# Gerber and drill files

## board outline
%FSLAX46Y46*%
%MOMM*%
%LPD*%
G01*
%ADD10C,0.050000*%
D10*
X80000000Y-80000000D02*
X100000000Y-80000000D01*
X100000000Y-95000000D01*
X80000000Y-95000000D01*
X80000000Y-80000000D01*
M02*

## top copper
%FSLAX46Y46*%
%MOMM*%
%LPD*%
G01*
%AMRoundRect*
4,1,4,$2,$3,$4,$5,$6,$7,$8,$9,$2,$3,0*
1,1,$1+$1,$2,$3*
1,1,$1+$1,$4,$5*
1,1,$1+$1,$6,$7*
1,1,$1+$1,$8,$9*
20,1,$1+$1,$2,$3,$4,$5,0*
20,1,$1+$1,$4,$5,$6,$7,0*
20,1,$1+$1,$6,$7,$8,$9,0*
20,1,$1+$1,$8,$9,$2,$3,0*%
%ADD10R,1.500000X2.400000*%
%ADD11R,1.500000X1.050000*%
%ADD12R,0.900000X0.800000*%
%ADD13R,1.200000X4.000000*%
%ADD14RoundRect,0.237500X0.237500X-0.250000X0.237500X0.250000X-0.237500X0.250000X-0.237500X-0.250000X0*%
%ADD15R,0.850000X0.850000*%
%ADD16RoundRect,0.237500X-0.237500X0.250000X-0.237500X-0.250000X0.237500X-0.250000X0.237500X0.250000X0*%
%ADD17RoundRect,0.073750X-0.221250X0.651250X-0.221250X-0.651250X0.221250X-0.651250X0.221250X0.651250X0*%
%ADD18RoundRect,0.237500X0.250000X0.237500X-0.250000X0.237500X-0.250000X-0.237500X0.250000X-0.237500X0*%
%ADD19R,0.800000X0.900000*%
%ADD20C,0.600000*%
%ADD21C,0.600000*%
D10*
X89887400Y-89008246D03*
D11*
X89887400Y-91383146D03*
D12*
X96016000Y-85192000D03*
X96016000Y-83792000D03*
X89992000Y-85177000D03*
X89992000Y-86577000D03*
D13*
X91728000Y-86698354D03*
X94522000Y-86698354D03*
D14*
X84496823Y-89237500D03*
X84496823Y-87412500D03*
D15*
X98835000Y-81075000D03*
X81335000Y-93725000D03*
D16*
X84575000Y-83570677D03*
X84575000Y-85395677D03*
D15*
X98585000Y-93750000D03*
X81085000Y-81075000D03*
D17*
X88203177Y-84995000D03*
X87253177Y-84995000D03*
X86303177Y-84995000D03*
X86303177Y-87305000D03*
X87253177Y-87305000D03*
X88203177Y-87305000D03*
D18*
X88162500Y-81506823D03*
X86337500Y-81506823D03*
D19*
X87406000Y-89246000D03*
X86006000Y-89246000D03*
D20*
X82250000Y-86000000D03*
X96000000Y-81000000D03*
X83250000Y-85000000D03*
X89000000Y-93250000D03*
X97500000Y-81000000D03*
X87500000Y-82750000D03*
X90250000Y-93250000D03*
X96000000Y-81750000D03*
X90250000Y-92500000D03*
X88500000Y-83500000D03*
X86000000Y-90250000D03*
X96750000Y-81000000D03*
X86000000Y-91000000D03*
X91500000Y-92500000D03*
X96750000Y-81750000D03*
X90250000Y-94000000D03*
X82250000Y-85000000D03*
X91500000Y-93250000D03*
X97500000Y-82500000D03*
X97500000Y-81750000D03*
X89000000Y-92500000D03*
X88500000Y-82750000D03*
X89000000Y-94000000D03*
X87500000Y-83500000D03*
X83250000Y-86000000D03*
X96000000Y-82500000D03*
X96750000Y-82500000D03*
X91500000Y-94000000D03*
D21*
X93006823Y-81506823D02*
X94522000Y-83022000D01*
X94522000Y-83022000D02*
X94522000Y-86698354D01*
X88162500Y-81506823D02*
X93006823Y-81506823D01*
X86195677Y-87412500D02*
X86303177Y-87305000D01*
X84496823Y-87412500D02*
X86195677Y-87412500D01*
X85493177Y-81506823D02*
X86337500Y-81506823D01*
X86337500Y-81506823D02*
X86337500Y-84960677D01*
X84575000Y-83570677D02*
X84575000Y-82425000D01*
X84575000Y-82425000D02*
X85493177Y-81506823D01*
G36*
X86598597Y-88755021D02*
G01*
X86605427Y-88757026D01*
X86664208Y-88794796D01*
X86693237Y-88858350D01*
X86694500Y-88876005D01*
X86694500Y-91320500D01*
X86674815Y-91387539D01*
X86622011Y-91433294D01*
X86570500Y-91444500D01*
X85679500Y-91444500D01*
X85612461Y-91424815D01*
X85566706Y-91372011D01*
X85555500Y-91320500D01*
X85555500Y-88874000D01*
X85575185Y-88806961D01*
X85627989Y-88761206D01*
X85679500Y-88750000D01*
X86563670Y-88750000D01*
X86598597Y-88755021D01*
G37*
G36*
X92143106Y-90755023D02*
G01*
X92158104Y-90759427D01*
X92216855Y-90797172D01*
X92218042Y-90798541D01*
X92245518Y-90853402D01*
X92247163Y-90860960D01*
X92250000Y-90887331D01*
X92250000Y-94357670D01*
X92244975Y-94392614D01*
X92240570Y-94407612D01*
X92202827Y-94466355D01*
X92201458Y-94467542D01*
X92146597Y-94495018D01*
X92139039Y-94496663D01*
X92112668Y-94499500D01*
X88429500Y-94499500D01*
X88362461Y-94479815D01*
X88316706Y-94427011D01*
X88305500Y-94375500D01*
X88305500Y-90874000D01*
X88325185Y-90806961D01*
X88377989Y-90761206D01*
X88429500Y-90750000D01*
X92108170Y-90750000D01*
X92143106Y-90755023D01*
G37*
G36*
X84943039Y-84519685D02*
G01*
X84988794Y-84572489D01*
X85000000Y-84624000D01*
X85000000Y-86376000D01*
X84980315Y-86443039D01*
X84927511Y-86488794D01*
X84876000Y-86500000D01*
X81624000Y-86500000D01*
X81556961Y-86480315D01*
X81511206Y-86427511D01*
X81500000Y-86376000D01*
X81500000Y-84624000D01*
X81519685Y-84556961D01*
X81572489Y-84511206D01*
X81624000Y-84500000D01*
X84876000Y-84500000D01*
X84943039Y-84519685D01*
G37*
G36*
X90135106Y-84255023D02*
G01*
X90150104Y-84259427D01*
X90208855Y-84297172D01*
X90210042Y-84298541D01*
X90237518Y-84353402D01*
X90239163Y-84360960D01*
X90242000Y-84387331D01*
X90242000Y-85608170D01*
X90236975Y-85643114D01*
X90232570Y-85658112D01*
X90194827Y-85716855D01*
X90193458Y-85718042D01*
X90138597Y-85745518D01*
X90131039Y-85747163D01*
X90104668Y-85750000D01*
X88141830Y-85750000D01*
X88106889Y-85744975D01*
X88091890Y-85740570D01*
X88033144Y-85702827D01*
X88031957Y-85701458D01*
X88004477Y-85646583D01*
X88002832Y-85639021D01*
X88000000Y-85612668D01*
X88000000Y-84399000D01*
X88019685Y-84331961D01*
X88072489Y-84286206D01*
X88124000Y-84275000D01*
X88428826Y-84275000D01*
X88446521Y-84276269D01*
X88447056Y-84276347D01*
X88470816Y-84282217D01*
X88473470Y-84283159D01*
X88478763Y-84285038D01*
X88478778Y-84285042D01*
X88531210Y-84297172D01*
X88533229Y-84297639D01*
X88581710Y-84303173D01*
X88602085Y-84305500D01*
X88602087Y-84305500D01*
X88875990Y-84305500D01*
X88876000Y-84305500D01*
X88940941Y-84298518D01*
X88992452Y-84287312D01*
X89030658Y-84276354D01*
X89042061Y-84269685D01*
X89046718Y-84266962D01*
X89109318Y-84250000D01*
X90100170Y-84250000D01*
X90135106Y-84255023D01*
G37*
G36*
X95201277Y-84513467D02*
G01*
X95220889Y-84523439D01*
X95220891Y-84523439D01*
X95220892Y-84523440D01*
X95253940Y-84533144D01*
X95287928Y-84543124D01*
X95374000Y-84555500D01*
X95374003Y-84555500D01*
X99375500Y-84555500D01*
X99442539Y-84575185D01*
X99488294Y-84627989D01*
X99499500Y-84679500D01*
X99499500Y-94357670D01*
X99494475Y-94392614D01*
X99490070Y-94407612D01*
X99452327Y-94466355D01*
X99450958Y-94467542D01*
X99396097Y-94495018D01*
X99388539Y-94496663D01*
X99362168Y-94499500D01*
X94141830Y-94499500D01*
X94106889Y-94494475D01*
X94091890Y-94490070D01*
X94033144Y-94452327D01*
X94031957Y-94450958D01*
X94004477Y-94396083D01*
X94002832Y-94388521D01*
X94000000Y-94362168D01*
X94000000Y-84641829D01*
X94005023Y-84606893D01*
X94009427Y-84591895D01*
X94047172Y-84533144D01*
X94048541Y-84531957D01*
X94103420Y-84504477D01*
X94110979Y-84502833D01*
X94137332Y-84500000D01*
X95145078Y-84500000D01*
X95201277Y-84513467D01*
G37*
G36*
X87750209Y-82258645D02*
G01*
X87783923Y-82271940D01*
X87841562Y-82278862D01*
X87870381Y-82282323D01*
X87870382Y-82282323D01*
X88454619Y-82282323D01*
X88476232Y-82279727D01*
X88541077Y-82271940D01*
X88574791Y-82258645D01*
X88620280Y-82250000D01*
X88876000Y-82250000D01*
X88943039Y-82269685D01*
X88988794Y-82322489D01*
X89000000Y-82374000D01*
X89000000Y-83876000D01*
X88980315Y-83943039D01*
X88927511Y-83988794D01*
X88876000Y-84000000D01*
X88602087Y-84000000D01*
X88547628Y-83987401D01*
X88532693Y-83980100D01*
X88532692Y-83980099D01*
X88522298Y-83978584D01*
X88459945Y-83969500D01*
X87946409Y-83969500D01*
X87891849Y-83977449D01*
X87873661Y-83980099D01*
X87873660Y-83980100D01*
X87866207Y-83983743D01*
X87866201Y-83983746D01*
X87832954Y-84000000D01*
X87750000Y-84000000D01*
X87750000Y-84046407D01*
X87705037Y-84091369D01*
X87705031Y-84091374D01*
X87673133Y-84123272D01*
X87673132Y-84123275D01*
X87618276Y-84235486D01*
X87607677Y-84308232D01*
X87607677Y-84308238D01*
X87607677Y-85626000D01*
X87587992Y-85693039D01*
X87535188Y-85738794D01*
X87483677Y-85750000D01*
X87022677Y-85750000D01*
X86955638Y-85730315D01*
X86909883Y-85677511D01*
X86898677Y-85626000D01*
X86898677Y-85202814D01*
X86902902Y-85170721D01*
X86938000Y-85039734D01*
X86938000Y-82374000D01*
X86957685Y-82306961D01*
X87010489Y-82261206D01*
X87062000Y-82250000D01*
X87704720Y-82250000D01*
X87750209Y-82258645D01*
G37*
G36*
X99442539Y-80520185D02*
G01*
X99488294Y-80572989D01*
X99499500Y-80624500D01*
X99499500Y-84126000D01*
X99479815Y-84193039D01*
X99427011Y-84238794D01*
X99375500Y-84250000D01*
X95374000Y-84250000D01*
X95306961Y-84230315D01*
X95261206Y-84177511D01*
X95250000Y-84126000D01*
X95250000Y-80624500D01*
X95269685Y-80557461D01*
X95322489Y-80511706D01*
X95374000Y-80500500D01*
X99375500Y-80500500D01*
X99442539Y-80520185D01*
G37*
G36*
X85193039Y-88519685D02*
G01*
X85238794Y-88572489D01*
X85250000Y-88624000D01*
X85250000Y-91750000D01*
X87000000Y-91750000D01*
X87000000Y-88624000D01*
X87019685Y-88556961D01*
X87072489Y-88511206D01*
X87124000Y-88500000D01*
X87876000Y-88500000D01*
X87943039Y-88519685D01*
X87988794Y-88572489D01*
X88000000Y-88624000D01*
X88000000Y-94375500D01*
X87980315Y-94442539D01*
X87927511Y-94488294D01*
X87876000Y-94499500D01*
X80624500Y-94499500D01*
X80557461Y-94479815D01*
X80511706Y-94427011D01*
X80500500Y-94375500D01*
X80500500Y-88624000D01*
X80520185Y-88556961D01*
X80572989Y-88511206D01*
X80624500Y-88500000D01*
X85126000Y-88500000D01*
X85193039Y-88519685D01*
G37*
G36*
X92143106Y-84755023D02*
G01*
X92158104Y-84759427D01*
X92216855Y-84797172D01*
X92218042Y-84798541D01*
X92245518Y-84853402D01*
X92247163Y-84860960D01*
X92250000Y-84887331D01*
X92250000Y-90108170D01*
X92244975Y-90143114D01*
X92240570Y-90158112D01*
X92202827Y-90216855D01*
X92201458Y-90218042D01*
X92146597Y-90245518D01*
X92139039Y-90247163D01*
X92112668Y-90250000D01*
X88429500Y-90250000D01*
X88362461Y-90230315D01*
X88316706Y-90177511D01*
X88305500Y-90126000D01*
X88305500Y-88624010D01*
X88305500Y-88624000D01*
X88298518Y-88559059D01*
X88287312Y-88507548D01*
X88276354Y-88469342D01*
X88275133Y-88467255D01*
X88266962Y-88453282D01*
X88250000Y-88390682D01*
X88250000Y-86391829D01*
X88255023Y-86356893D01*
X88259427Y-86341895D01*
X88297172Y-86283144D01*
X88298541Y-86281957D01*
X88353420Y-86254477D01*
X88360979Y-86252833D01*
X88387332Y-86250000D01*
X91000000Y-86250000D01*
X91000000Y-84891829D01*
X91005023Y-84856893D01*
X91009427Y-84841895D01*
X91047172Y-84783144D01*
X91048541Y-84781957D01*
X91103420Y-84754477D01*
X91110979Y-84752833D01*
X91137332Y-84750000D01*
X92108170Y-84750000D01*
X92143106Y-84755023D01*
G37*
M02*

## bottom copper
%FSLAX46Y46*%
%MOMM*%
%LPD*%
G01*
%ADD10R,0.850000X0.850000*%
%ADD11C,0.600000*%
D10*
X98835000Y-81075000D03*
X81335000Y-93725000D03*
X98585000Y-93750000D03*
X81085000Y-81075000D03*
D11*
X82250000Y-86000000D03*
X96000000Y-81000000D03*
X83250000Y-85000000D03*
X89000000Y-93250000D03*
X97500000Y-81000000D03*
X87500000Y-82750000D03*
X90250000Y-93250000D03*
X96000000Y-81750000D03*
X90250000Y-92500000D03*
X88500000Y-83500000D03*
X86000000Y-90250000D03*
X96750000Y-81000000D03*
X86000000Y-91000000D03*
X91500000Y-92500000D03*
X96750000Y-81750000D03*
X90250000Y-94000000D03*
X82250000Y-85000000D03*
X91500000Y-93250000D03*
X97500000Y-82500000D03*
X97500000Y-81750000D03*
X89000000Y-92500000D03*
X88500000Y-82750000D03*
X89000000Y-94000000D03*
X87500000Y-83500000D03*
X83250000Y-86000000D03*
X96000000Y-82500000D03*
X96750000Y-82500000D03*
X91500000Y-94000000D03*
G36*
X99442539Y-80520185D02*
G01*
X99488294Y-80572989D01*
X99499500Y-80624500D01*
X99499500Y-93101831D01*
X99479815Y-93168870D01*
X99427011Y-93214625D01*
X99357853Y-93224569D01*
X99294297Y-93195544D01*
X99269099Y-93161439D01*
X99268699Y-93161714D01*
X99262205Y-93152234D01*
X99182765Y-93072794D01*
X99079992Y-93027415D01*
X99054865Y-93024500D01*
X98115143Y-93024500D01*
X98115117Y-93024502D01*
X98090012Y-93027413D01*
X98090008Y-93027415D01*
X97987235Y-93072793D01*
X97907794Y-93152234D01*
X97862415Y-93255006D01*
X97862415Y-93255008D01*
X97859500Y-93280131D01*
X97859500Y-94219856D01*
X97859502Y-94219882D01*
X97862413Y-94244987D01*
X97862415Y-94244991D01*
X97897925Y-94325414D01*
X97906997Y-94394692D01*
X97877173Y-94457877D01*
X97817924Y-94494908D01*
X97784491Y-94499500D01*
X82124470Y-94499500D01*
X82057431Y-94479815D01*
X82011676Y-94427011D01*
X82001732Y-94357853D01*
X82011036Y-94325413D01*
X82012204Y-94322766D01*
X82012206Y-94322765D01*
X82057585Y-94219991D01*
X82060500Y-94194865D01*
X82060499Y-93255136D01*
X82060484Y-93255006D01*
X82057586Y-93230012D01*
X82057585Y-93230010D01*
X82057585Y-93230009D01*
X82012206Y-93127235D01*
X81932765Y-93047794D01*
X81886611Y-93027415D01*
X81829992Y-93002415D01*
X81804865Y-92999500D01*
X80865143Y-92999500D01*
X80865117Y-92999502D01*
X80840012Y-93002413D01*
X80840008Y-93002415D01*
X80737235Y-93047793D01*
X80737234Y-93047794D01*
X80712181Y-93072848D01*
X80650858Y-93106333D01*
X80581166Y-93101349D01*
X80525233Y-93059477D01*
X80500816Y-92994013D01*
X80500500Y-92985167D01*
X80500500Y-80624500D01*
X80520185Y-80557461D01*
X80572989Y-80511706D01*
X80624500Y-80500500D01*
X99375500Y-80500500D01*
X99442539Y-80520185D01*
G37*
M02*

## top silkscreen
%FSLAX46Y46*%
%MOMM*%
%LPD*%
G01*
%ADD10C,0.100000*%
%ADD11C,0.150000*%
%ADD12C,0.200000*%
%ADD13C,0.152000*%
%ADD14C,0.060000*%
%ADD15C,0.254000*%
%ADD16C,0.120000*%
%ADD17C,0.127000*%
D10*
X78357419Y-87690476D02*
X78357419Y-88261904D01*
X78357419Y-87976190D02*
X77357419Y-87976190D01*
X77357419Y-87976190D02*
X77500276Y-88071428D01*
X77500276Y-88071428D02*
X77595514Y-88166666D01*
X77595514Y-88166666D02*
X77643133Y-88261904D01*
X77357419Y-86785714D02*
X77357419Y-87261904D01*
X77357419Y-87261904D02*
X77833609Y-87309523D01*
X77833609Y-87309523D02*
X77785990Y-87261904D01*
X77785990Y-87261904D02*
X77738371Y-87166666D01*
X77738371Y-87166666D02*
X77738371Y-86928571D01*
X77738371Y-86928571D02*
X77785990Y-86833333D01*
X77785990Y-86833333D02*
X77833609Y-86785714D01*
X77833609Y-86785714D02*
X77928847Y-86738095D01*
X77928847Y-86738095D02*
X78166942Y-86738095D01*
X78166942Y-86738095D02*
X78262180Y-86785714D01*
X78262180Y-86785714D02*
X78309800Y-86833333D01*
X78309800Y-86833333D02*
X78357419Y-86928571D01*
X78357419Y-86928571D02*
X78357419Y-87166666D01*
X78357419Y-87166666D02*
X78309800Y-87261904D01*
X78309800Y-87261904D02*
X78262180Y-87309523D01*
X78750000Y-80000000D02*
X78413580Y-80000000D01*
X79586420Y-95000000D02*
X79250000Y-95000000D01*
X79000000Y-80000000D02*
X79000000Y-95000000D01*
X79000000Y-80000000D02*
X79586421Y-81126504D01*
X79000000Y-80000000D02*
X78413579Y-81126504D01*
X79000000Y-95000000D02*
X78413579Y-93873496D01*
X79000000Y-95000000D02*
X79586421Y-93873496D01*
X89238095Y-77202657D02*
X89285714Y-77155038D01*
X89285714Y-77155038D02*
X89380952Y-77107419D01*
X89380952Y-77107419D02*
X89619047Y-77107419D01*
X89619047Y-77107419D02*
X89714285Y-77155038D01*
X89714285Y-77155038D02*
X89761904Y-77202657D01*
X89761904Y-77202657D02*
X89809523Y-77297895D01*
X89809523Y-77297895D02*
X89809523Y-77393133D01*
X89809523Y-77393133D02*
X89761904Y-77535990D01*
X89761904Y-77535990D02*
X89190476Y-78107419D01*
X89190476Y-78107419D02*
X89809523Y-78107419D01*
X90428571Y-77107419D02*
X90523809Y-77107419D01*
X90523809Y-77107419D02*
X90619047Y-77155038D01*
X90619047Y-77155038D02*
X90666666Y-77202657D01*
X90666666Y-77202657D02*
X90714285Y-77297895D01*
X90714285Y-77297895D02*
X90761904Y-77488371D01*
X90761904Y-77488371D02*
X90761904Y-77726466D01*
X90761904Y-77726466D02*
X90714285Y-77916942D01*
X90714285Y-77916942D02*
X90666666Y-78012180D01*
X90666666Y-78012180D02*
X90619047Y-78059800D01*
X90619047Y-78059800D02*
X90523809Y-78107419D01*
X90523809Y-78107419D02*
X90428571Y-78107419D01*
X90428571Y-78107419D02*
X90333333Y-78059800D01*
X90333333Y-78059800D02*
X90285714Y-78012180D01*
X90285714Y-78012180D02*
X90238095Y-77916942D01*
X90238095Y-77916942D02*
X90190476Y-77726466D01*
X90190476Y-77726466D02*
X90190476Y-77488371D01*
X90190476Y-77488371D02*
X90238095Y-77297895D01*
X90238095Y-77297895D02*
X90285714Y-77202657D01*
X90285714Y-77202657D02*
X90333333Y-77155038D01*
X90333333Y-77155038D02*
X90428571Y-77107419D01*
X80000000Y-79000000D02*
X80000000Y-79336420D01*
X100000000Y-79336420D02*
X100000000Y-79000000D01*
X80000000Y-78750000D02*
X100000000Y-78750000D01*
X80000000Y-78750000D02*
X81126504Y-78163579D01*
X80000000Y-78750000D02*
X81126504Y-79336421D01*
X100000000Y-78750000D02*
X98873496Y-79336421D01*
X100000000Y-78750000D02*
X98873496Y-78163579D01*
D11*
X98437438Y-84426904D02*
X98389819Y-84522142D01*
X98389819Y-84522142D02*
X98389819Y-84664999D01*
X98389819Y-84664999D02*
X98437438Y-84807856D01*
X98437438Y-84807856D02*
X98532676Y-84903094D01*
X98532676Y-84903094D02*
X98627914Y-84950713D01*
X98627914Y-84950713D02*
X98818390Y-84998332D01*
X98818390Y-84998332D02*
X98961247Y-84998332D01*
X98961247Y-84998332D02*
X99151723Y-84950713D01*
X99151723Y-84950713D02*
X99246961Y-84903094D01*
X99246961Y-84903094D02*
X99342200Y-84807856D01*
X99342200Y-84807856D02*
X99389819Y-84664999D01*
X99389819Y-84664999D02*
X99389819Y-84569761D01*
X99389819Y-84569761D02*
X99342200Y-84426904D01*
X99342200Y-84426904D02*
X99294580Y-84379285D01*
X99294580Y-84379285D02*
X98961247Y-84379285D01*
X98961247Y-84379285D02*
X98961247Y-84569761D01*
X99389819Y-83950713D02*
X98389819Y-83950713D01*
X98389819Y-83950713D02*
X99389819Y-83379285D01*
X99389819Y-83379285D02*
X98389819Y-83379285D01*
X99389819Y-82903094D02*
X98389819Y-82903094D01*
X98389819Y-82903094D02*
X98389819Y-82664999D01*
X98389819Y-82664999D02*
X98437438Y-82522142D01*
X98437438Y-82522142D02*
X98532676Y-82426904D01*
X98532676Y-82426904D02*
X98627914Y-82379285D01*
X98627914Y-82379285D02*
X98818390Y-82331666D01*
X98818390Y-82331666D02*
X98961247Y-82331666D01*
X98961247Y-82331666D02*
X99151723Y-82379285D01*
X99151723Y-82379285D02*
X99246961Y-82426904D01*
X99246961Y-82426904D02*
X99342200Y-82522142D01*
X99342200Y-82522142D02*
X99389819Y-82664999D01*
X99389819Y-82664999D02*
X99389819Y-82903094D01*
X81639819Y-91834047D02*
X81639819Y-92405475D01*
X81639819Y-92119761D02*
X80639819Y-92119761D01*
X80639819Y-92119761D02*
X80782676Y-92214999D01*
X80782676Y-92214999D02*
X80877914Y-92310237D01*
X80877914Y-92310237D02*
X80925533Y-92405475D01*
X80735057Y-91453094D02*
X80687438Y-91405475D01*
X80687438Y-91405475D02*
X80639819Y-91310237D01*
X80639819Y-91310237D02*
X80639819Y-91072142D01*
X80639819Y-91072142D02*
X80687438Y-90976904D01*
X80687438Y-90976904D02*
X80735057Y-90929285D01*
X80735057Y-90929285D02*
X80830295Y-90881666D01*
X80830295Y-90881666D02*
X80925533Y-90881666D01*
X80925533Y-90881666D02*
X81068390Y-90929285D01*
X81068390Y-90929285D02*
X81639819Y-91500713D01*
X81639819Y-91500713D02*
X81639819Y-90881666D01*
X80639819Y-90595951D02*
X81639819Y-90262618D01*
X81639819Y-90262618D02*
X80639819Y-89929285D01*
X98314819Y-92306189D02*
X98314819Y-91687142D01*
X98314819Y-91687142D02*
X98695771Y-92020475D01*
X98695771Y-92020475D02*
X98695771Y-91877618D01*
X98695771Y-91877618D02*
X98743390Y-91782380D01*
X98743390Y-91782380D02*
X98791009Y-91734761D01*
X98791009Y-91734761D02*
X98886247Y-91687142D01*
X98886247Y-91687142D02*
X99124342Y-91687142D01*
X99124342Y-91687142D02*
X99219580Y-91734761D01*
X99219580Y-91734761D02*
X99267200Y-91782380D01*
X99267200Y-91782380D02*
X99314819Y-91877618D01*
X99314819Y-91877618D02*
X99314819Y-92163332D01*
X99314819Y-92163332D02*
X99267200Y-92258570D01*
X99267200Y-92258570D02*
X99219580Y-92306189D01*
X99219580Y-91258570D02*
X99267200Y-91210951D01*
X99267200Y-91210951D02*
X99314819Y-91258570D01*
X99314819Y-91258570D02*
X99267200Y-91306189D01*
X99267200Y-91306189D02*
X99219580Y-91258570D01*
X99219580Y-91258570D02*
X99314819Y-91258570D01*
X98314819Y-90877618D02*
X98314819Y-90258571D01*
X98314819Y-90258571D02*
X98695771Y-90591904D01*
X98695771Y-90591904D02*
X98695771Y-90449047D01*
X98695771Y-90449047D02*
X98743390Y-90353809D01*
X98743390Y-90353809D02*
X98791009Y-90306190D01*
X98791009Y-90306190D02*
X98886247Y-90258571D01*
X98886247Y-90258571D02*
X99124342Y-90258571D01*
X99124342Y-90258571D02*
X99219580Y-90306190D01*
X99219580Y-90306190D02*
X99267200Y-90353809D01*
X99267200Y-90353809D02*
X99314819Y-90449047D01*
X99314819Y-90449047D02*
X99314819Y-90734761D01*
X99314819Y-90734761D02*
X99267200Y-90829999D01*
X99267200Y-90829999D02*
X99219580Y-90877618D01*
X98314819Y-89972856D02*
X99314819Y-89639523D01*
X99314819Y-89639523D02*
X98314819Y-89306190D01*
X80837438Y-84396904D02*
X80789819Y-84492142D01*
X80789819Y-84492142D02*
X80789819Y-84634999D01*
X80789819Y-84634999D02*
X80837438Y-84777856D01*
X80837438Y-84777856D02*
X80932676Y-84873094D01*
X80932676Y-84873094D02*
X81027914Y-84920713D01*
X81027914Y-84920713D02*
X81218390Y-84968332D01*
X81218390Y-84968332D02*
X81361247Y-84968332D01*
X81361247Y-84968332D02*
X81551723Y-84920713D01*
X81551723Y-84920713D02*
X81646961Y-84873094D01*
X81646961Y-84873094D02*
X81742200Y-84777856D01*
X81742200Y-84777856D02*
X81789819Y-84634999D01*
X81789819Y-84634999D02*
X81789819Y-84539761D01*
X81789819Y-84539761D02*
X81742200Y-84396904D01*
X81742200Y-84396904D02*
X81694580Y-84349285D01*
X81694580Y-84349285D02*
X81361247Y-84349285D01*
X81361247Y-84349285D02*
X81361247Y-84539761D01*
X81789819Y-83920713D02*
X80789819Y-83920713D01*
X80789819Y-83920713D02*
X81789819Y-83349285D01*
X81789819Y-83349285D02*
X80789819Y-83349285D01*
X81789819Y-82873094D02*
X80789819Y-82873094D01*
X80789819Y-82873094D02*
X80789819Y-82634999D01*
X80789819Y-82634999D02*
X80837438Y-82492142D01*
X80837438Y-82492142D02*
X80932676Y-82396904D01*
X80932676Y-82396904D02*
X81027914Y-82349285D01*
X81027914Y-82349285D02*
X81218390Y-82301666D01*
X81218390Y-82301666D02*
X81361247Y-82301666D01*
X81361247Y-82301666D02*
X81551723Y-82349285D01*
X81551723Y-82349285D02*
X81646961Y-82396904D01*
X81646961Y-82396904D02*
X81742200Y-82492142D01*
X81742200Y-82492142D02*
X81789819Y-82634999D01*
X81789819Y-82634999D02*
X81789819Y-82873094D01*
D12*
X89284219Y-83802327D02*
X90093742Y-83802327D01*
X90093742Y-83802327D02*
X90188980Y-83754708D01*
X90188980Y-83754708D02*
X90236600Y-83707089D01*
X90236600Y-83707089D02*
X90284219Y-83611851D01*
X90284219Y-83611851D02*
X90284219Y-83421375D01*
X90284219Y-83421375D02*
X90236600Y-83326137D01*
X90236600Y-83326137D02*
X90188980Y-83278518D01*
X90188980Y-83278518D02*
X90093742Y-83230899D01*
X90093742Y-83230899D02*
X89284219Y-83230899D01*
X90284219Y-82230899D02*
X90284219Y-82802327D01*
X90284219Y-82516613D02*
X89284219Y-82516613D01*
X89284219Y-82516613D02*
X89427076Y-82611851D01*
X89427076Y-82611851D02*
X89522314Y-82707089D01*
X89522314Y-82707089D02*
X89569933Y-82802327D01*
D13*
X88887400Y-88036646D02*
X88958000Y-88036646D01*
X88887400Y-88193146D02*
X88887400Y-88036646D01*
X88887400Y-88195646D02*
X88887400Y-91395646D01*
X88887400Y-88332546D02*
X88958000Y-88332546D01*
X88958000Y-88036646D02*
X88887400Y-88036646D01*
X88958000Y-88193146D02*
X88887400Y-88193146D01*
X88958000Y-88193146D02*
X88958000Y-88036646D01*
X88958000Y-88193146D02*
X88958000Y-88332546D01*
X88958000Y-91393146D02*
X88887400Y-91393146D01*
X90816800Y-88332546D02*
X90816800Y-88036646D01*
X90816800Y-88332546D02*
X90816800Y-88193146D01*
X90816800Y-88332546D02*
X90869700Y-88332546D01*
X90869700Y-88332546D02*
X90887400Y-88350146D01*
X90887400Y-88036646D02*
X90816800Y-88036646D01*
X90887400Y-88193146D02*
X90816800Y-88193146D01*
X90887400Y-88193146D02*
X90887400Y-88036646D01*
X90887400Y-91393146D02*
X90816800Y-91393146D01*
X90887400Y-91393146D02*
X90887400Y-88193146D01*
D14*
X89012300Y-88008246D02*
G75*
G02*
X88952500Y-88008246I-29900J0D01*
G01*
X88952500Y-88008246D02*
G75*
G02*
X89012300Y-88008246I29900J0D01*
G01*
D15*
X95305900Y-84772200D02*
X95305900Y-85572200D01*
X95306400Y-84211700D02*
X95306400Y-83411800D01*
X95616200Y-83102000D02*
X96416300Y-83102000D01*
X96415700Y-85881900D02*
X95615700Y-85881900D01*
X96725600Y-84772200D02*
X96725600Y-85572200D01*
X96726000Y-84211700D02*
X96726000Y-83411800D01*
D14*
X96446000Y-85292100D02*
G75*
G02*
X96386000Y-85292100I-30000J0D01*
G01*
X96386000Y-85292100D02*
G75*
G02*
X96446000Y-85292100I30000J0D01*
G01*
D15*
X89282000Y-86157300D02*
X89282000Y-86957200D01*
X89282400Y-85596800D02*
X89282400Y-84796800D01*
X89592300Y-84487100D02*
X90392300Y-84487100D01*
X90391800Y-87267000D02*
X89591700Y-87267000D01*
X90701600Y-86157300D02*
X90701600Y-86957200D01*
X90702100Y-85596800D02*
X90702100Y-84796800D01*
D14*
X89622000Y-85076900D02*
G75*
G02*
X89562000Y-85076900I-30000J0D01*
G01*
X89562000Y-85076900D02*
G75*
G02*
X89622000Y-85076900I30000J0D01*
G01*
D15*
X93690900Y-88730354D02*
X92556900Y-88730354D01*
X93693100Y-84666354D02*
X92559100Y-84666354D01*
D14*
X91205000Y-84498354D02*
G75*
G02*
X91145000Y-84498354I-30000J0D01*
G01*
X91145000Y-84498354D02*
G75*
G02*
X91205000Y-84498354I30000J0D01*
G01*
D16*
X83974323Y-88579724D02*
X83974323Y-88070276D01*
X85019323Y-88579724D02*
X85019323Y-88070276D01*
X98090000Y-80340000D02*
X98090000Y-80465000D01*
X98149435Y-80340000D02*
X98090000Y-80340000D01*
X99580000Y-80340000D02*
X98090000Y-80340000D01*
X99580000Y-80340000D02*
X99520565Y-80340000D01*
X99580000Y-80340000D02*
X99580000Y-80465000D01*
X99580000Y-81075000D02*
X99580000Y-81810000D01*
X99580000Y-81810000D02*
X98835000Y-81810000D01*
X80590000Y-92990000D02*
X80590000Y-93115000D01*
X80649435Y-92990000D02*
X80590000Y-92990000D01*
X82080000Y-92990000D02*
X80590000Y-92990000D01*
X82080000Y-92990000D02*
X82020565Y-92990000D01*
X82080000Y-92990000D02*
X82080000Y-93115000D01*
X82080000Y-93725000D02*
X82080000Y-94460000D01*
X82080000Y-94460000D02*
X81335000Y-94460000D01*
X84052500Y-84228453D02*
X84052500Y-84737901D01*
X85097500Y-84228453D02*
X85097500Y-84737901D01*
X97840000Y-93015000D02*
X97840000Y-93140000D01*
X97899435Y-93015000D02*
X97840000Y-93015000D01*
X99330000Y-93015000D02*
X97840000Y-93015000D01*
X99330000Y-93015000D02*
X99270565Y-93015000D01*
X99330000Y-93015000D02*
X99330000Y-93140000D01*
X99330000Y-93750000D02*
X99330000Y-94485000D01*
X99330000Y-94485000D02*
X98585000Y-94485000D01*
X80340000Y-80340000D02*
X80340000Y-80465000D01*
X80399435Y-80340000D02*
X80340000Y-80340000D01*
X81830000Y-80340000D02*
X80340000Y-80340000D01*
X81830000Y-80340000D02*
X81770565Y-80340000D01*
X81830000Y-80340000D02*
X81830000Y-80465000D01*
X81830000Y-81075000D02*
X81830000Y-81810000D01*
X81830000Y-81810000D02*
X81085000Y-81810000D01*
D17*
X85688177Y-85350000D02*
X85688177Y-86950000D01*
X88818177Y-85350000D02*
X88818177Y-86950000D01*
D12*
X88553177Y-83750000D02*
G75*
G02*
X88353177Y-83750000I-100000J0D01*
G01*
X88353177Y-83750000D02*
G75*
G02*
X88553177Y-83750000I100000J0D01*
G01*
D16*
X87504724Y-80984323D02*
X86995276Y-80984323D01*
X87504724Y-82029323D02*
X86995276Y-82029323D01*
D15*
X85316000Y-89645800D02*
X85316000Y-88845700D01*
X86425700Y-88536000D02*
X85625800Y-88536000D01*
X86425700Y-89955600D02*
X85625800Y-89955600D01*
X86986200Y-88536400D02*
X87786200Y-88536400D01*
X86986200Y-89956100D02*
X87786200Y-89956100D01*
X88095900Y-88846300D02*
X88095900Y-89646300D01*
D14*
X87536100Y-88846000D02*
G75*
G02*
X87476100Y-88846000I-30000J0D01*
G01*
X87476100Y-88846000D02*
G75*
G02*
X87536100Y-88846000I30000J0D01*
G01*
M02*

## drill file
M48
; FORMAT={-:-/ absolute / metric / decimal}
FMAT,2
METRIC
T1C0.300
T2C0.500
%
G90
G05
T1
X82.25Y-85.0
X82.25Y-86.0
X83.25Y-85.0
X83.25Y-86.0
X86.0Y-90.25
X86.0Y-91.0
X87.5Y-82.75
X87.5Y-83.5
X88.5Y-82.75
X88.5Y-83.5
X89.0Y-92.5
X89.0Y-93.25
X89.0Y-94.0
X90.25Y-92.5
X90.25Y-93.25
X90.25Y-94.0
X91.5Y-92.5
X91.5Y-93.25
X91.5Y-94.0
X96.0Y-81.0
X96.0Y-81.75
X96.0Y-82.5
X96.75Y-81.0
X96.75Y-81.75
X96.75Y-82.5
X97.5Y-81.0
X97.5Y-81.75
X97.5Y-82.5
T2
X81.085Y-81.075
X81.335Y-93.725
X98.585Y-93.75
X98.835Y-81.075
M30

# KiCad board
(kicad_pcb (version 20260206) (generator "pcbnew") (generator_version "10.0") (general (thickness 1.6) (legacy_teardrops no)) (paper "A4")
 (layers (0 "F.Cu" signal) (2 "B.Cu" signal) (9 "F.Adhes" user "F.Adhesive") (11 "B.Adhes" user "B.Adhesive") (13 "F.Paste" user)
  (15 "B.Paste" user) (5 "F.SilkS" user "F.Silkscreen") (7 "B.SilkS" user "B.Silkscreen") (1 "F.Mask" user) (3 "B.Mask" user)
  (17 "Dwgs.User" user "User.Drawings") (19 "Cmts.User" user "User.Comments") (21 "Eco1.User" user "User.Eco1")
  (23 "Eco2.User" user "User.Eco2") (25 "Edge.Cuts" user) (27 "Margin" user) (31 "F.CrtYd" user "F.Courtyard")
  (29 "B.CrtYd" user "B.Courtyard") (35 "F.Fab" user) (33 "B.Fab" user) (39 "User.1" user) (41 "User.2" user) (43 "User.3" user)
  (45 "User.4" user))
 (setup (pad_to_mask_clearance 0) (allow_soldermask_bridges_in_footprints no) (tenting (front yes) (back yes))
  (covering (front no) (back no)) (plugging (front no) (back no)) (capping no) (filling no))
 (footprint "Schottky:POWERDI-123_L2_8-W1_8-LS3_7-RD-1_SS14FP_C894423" (layer "F.Cu") (at 89.8874 90.195646 -90)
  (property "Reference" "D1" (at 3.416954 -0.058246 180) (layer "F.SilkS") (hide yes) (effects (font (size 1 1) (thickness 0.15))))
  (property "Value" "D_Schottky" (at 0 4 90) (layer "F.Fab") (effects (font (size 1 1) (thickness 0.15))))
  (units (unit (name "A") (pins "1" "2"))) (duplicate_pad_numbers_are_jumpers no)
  (fp_line (start -2.159 1) (end -2.159 0.9294) (stroke (width 0.152) (type solid)) (layer "F.SilkS"))
  (fp_line (start -2.0025 1) (end -2.159 1) (stroke (width 0.152) (type solid)) (layer "F.SilkS"))
  (fp_line (start -2 1) (end 1.2 1) (stroke (width 0.152) (type solid)) (layer "F.SilkS"))
  (fp_line (start -1.8631 1) (end -1.8631 0.9294) (stroke (width 0.152) (type solid)) (layer "F.SilkS"))
  (fp_line (start -2.159 0.9294) (end -2.159 1) (stroke (width 0.152) (type solid)) (layer "F.SilkS"))
  (fp_line (start -2.0025 0.9294) (end -2.0025 1) (stroke (width 0.152) (type solid)) (layer "F.SilkS"))
  (fp_line (start -2.0025 0.9294) (end -2.159 0.9294) (stroke (width 0.152) (type solid)) (layer "F.SilkS"))
  (fp_line (start -2.0025 0.9294) (end -1.8631 0.9294) (stroke (width 0.152) (type solid)) (layer "F.SilkS"))
  (fp_line (start 1.1975 0.9294) (end 1.1975 1) (stroke (width 0.152) (type solid)) (layer "F.SilkS"))
  (fp_line (start -1.8631 -0.9294) (end -2.159 -0.9294) (stroke (width 0.152) (type solid)) (layer "F.SilkS"))
  (fp_line (start -1.8631 -0.9294) (end -2.0025 -0.9294) (stroke (width 0.152) (type solid)) (layer "F.SilkS"))
  (fp_line (start -1.8631 -0.9294) (end -1.8631 -0.9823) (stroke (width 0.152) (type solid)) (layer "F.SilkS"))
  (fp_line (start -1.8631 -0.9823) (end -1.8455 -1) (stroke (width 0.152) (type solid)) (layer "F.SilkS"))
  (fp_line (start -2.159 -1) (end -2.159 -0.9294) (stroke (width 0.152) (type solid)) (layer "F.SilkS"))
  (fp_line (start -2.0025 -1) (end -2.0025 -0.9294) (stroke (width 0.152) (type solid)) (layer "F.SilkS"))
  (fp_line (start -2.0025 -1) (end -2.159 -1) (stroke (width 0.152) (type solid)) (layer "F.SilkS"))
  (fp_line (start 1.1975 -1) (end 1.1975 -0.9294) (stroke (width 0.152) (type solid)) (layer "F.SilkS"))
  (fp_line (start 1.1975 -1) (end -2.0025 -1) (stroke (width 0.152) (type solid)) (layer "F.SilkS"))
  (fp_circle (center -2.1874 0.905) (end -2.1575 0.905) (stroke (width 0.06) (type solid)) (fill no) (layer "F.SilkS"))
  (pad "1" smd rect (at -1.1874 0 90) (size 2.4 1.5) (layers "F.Cu" "F.Mask" "F.Paste") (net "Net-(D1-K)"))
  (pad "2" smd rect (at 1.1875 0 90) (size 1.05 1.5) (layers "F.Cu" "F.Mask" "F.Paste") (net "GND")))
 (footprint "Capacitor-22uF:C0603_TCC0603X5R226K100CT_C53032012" (layer "F.Cu") (at 96.016 84.492 90)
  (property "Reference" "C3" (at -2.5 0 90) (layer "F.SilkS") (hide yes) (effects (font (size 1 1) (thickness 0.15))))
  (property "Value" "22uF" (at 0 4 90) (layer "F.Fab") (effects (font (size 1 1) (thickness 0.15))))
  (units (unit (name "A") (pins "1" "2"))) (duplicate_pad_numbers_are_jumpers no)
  (fp_line (start -0.2802 -0.7101) (end -1.0802 -0.7101) (stroke (width 0.254) (type solid)) (layer "F.SilkS"))
  (fp_line (start 0.2803 -0.7096) (end 1.0802 -0.7096) (stroke (width 0.254) (type solid)) (layer "F.SilkS"))
  (fp_line (start 1.39 -0.3998) (end 1.39 0.4003) (stroke (width 0.254) (type solid)) (layer "F.SilkS"))
  (fp_line (start -1.3899 0.3997) (end -1.3899 -0.4003) (stroke (width 0.254) (type solid)) (layer "F.SilkS"))
  (fp_line (start -0.2802 0.7096) (end -1.0802 0.7096) (stroke (width 0.254) (type solid)) (layer "F.SilkS"))
  (fp_line (start 0.2803 0.71) (end 1.0802 0.71) (stroke (width 0.254) (type solid)) (layer "F.SilkS"))
  (fp_circle (center -0.8001 0.4) (end -0.7701 0.4) (stroke (width 0.06) (type solid)) (fill no) (layer "F.SilkS"))
  (pad "1" smd rect (at -0.7 0 90) (size 0.8 0.9) (layers "F.Cu" "F.Mask" "F.Paste") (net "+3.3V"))
  (pad "2" smd rect (at 0.7 0 90) (size 0.8 0.9) (layers "F.Cu" "F.Mask" "F.Paste") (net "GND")))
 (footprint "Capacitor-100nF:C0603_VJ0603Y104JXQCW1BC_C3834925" (layer "F.Cu") (at 89.992 85.877 -90)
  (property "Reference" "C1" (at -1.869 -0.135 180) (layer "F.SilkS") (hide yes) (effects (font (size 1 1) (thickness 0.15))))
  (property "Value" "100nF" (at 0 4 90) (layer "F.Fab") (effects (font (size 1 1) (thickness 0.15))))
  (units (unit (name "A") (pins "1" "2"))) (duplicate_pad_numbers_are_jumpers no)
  (fp_line (start 0.2803 0.71) (end 1.0802 0.71) (stroke (width 0.254) (type solid)) (layer "F.SilkS"))
  (fp_line (start -0.2802 0.7096) (end -1.0802 0.7096) (stroke (width 0.254) (type solid)) (layer "F.SilkS"))
  (fp_line (start -1.3899 0.3997) (end -1.3899 -0.4003) (stroke (width 0.254) (type solid)) (layer "F.SilkS"))
  (fp_line (start 1.39 -0.3998) (end 1.39 0.4003) (stroke (width 0.254) (type solid)) (layer "F.SilkS"))
  (fp_line (start 0.2803 -0.7096) (end 1.0802 -0.7096) (stroke (width 0.254) (type solid)) (layer "F.SilkS"))
  (fp_line (start -0.2802 -0.7101) (end -1.0802 -0.7101) (stroke (width 0.254) (type solid)) (layer "F.SilkS"))
  (fp_circle (center -0.8001 0.4) (end -0.7701 0.4) (stroke (width 0.06) (type solid)) (fill no) (layer "F.SilkS"))
  (pad "1" smd rect (at -0.7 0 270) (size 0.8 0.9) (layers "F.Cu" "F.Mask" "F.Paste") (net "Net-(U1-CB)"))
  (pad "2" smd rect (at 0.7 0 270) (size 0.8 0.9) (layers "F.Cu" "F.Mask" "F.Paste") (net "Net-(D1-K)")))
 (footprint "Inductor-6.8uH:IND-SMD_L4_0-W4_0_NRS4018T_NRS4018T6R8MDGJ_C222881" (layer "F.Cu") (at 93.125 86.698354 180)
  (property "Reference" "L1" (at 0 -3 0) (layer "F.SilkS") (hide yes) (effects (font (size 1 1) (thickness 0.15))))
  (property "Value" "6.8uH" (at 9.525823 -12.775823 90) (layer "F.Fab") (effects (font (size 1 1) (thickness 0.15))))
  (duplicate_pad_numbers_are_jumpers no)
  (fp_line (start -0.5659 -2.032) (end 0.5681 -2.032) (stroke (width 0.254) (type solid)) (layer "F.SilkS"))
  (fp_line (start -0.5681 2.032) (end 0.5659 2.032) (stroke (width 0.254) (type solid)) (layer "F.SilkS"))
  (fp_circle (center 1.95 2.2) (end 1.98 2.2) (stroke (width 0.06) (type solid)) (fill no) (layer "F.SilkS"))
  (pad "1" smd rect (at 1.397 0 180) (size 1.2 4) (layers "F.Cu" "F.Mask" "F.Paste") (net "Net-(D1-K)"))
  (pad "2" smd rect (at -1.397 0 180) (size 1.2 4) (layers "F.Cu" "F.Mask" "F.Paste") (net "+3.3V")))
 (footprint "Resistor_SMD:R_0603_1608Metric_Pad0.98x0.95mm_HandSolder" (layer "F.Cu") (at 84.496823 88.325 90)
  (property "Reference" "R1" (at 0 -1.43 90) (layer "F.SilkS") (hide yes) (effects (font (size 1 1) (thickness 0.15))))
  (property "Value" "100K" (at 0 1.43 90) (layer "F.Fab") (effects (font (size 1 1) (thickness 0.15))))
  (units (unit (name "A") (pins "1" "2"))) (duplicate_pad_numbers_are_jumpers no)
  (fp_line (start -0.254724 -0.5225) (end 0.254724 -0.5225) (stroke (width 0.12) (type solid)) (layer "F.SilkS"))
  (fp_line (start -0.254724 0.5225) (end 0.254724 0.5225) (stroke (width 0.12) (type solid)) (layer "F.SilkS"))
  (pad "1" smd roundrect (at -0.9125 0 90) (size 0.975 0.95) (layers "F.Cu" "F.Mask" "F.Paste") (roundrect_rratio 0.25) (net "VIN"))
  (pad "2" smd roundrect (at 0.9125 0 90) (size 0.975 0.95) (layers "F.Cu" "F.Mask" "F.Paste") (roundrect_rratio 0.25) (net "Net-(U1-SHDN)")))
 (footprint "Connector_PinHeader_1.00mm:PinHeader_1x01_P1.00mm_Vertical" (layer "F.Cu") (at 98.835 81.075 180)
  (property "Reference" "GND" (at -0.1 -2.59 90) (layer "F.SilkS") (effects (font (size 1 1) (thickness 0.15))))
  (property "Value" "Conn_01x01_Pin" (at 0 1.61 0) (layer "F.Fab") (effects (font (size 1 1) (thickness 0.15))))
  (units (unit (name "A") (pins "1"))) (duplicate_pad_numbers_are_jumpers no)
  (fp_line (start 0.745 0.735) (end 0.745 0.61) (stroke (width 0.12) (type solid)) (layer "F.SilkS"))
  (fp_line (start 0.685565 0.735) (end 0.745 0.735) (stroke (width 0.12) (type solid)) (layer "F.SilkS"))
  (fp_line (start -0.745 0.735) (end 0.745 0.735) (stroke (width 0.12) (type solid)) (layer "F.SilkS"))
  (fp_line (start -0.745 0.735) (end -0.685565 0.735) (stroke (width 0.12) (type solid)) (layer "F.SilkS"))
  (fp_line (start -0.745 0.735) (end -0.745 0.61) (stroke (width 0.12) (type solid)) (layer "F.SilkS"))
  (fp_line (start -0.745 0) (end -0.745 -0.735) (stroke (width 0.12) (type solid)) (layer "F.SilkS"))
  (fp_line (start -0.745 -0.735) (end 0 -0.735) (stroke (width 0.12) (type solid)) (layer "F.SilkS"))
  (pad "1" thru_hole rect (at 0 0 180) (size 0.85 0.85) (drill 0.5) (layers "*.Cu" "*.Mask") (remove_unused_layers no) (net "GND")))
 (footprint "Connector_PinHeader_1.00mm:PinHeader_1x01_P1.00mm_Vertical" (layer "F.Cu") (at 81.335 93.725 180)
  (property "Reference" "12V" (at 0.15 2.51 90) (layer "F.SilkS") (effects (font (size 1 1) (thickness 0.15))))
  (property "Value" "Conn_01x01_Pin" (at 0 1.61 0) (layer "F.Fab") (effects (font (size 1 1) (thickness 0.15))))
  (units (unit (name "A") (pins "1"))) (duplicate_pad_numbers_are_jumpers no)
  (fp_line (start 0.745 0.735) (end 0.745 0.61) (stroke (width 0.12) (type solid)) (layer "F.SilkS"))
  (fp_line (start 0.685565 0.735) (end 0.745 0.735) (stroke (width 0.12) (type solid)) (layer "F.SilkS"))
  (fp_line (start -0.745 0.735) (end 0.745 0.735) (stroke (width 0.12) (type solid)) (layer "F.SilkS"))
  (fp_line (start -0.745 0.735) (end -0.685565 0.735) (stroke (width 0.12) (type solid)) (layer "F.SilkS"))
  (fp_line (start -0.745 0.735) (end -0.745 0.61) (stroke (width 0.12) (type solid)) (layer "F.SilkS"))
  (fp_line (start -0.745 0) (end -0.745 -0.735) (stroke (width 0.12) (type solid)) (layer "F.SilkS"))
  (fp_line (start -0.745 -0.735) (end 0 -0.735) (stroke (width 0.12) (type solid)) (layer "F.SilkS"))
  (pad "1" thru_hole rect (at 0 0 180) (size 0.85 0.85) (drill 0.5) (layers "*.Cu" "*.Mask") (remove_unused_layers no) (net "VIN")))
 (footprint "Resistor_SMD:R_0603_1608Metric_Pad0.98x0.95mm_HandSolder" (layer "F.Cu") (at 84.575 84.483177 -90)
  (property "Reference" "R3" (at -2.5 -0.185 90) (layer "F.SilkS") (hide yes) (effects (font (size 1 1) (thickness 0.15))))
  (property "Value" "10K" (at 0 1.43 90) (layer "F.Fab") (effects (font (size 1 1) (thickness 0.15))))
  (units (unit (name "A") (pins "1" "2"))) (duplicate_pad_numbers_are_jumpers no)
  (fp_line (start -0.254724 0.5225) (end 0.254724 0.5225) (stroke (width 0.12) (type solid)) (layer "F.SilkS"))
  (fp_line (start -0.254724 -0.5225) (end 0.254724 -0.5225) (stroke (width 0.12) (type solid)) (layer "F.SilkS"))
  (pad "1" smd roundrect (at -0.9125 0 270) (size 0.975 0.95) (layers "F.Cu" "F.Mask" "F.Paste") (roundrect_rratio 0.25) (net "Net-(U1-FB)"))
  (pad "2" smd roundrect (at 0.9125 0 270) (size 0.975 0.95) (layers "F.Cu" "F.Mask" "F.Paste") (roundrect_rratio 0.25) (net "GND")))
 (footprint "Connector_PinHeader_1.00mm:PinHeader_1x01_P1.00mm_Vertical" (layer "F.Cu") (at 98.585 93.75 180)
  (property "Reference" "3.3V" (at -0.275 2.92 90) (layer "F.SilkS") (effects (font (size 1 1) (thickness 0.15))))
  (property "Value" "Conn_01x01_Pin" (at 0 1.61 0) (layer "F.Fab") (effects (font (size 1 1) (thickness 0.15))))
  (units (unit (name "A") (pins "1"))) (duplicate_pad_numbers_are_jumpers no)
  (fp_line (start 0.745 0.735) (end 0.745 0.61) (stroke (width 0.12) (type solid)) (layer "F.SilkS"))
  (fp_line (start 0.685565 0.735) (end 0.745 0.735) (stroke (width 0.12) (type solid)) (layer "F.SilkS"))
  (fp_line (start -0.745 0.735) (end 0.745 0.735) (stroke (width 0.12) (type solid)) (layer "F.SilkS"))
  (fp_line (start -0.745 0.735) (end -0.685565 0.735) (stroke (width 0.12) (type solid)) (layer "F.SilkS"))
  (fp_line (start -0.745 0.735) (end -0.745 0.61) (stroke (width 0.12) (type solid)) (layer "F.SilkS"))
  (fp_line (start -0.745 0) (end -0.745 -0.735) (stroke (width 0.12) (type solid)) (layer "F.SilkS"))
  (fp_line (start -0.745 -0.735) (end 0 -0.735) (stroke (width 0.12) (type solid)) (layer "F.SilkS"))
  (pad "1" thru_hole rect (at 0 0 180) (size 0.85 0.85) (drill 0.5) (layers "*.Cu" "*.Mask") (remove_unused_layers no) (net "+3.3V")))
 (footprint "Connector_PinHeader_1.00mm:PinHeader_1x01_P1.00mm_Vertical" (layer "F.Cu") (at 81.085 81.075 180)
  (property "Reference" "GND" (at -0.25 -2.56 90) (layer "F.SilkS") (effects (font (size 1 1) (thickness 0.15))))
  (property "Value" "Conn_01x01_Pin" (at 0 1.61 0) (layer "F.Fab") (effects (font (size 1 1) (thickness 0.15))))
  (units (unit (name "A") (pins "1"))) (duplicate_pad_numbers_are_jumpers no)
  (fp_line (start 0.745 0.735) (end 0.745 0.61) (stroke (width 0.12) (type solid)) (layer "F.SilkS"))
  (fp_line (start 0.685565 0.735) (end 0.745 0.735) (stroke (width 0.12) (type solid)) (layer "F.SilkS"))
  (fp_line (start -0.745 0.735) (end 0.745 0.735) (stroke (width 0.12) (type solid)) (layer "F.SilkS"))
  (fp_line (start -0.745 0.735) (end -0.685565 0.735) (stroke (width 0.12) (type solid)) (layer "F.SilkS"))
  (fp_line (start -0.745 0.735) (end -0.745 0.61) (stroke (width 0.12) (type solid)) (layer "F.SilkS"))
  (fp_line (start -0.745 0) (end -0.745 -0.735) (stroke (width 0.12) (type solid)) (layer "F.SilkS"))
  (fp_line (start -0.745 -0.735) (end 0 -0.735) (stroke (width 0.12) (type solid)) (layer "F.SilkS"))
  (pad "1" thru_hole rect (at 0 0 180) (size 0.85 0.85) (drill 0.5) (layers "*.Cu" "*.Mask") (remove_unused_layers no) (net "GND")))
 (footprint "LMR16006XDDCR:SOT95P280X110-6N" (layer "F.Cu") (at 87.253177 86.15 -90)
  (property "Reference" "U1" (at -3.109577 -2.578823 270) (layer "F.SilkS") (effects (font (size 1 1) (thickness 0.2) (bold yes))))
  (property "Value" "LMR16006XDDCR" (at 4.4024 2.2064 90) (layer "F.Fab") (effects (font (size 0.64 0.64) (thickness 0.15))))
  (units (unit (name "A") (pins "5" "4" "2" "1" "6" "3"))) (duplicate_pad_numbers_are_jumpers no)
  (fp_line (start -0.8 1.565) (end 0.8 1.565) (stroke (width 0.127) (type solid)) (layer "F.SilkS"))
  (fp_line (start -0.8 -1.565) (end 0.8 -1.565) (stroke (width 0.127) (type solid)) (layer "F.SilkS"))
  (fp_circle (center -2.4 -1.2) (end -2.3 -1.2) (stroke (width 0.2) (type solid)) (fill no) (layer "F.SilkS"))
  (pad "1" smd roundrect (at -1.155 -0.95 270) (size 1.45 0.59) (layers "F.Cu" "F.Mask" "F.Paste") (roundrect_rratio 0.125)
   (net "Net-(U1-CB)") (solder_mask_margin 0.102))
  (pad "2" smd roundrect (at -1.155 0 270) (size 1.45 0.59) (layers "F.Cu" "F.Mask" "F.Paste") (roundrect_rratio 0.125) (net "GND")
   (solder_mask_margin 0.102))
  (pad "3" smd roundrect (at -1.155 0.95 270) (size 1.45 0.59) (layers "F.Cu" "F.Mask" "F.Paste") (roundrect_rratio 0.125)
   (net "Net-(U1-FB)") (solder_mask_margin 0.102))
  (pad "4" smd roundrect (at 1.155 0.95 270) (size 1.45 0.59) (layers "F.Cu" "F.Mask" "F.Paste") (roundrect_rratio 0.125)
   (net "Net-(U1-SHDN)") (solder_mask_margin 0.102))
  (pad "5" smd roundrect (at 1.155 0 270) (size 1.45 0.59) (layers "F.Cu" "F.Mask" "F.Paste") (roundrect_rratio 0.125) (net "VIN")
   (solder_mask_margin 0.102))
  (pad "6" smd roundrect (at 1.155 -0.95 270) (size 1.45 0.59) (layers "F.Cu" "F.Mask" "F.Paste") (roundrect_rratio 0.125)
   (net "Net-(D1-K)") (solder_mask_margin 0.102)))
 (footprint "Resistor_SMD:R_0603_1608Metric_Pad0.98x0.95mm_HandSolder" (layer "F.Cu") (at 87.25 81.506823 180)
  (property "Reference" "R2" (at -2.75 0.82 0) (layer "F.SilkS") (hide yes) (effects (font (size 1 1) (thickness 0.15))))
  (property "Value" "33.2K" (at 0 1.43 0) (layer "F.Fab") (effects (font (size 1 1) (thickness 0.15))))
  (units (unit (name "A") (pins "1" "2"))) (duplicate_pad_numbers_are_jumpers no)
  (fp_line (start -0.254724 0.5225) (end 0.254724 0.5225) (stroke (width 0.12) (type solid)) (layer "F.SilkS"))
  (fp_line (start -0.254724 -0.5225) (end 0.254724 -0.5225) (stroke (width 0.12) (type solid)) (layer "F.SilkS"))
  (pad "1" smd roundrect (at -0.9125 0 180) (size 0.975 0.95) (layers "F.Cu" "F.Mask" "F.Paste") (roundrect_rratio 0.25) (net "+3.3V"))
  (pad "2" smd roundrect (at 0.9125 0 180) (size 0.975 0.95) (layers "F.Cu" "F.Mask" "F.Paste") (roundrect_rratio 0.25) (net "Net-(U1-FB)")))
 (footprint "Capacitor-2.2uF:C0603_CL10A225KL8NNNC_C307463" (layer "F.Cu") (at 86.706 89.246 180)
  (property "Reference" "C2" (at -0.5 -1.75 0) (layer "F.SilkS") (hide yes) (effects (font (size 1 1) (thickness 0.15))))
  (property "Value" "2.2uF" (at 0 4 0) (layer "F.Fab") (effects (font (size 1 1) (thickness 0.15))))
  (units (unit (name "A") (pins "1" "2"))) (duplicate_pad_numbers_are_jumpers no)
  (fp_line (start 1.39 -0.3998) (end 1.39 0.4003) (stroke (width 0.254) (type solid)) (layer "F.SilkS"))
  (fp_line (start 0.2803 0.71) (end 1.0802 0.71) (stroke (width 0.254) (type solid)) (layer "F.SilkS"))
  (fp_line (start 0.2803 -0.7096) (end 1.0802 -0.7096) (stroke (width 0.254) (type solid)) (layer "F.SilkS"))
  (fp_line (start -0.2802 0.7096) (end -1.0802 0.7096) (stroke (width 0.254) (type solid)) (layer "F.SilkS"))
  (fp_line (start -0.2802 -0.7101) (end -1.0802 -0.7101) (stroke (width 0.254) (type solid)) (layer "F.SilkS"))
  (fp_line (start -1.3899 0.3997) (end -1.3899 -0.4003) (stroke (width 0.254) (type solid)) (layer "F.SilkS"))
  (fp_circle (center -0.8001 0.4) (end -0.7701 0.4) (stroke (width 0.06) (type solid)) (fill no) (layer "F.SilkS"))
  (pad "1" smd rect (at -0.7 0 180) (size 0.8 0.9) (layers "F.Cu" "F.Mask" "F.Paste") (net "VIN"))
  (pad "2" smd rect (at 0.7 0 180) (size 0.8 0.9) (layers "F.Cu" "F.Mask" "F.Paste") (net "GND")))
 (gr_rect (start 80 80) (end 100 95) (stroke (width 0.05) (type default)) (fill no) (layer "Edge.Cuts"))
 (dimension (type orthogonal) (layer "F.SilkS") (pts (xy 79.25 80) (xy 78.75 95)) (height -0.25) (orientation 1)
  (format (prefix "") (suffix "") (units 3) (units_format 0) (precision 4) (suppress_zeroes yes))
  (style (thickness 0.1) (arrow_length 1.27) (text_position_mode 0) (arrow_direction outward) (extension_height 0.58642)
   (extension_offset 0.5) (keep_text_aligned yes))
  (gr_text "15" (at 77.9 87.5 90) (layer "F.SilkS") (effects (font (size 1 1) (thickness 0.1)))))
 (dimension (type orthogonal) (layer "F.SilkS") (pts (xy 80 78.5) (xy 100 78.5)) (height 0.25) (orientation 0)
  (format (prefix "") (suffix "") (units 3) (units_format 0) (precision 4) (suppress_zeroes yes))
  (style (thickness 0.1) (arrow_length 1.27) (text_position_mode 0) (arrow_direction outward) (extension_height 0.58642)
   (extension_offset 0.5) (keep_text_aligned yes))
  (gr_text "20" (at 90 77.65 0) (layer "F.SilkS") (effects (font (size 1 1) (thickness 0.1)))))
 (via (at 82.25 86) (size 0.6) (drill 0.3) (layers "F.Cu" "B.Cu") (free yes) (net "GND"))
 (via (at 96 81) (size 0.6) (drill 0.3) (layers "F.Cu" "B.Cu") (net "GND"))
 (via (at 83.25 85) (size 0.6) (drill 0.3) (layers "F.Cu" "B.Cu") (free yes) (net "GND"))
 (via (at 89 93.25) (size 0.6) (drill 0.3) (layers "F.Cu" "B.Cu") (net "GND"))
 (via (at 97.5 81) (size 0.6) (drill 0.3) (layers "F.Cu" "B.Cu") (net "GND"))
 (via (at 87.5 82.75) (size 0.6) (drill 0.3) (layers "F.Cu" "B.Cu") (free yes) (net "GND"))
 (via (at 90.25 93.25) (size 0.6) (drill 0.3) (layers "F.Cu" "B.Cu") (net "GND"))
 (via (at 96 81.75) (size 0.6) (drill 0.3) (layers "F.Cu" "B.Cu") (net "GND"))
 (via (at 90.25 92.5) (size 0.6) (drill 0.3) (layers "F.Cu" "B.Cu") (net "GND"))
 (via (at 88.5 83.5) (size 0.6) (drill 0.3) (layers "F.Cu" "B.Cu") (free yes) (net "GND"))
 (via (at 86 90.25) (size 0.6) (drill 0.3) (layers "F.Cu" "B.Cu") (free yes) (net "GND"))
 (via (at 96.75 81) (size 0.6) (drill 0.3) (layers "F.Cu" "B.Cu") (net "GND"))
 (via (at 86 91) (size 0.6) (drill 0.3) (layers "F.Cu" "B.Cu") (free yes) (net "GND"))
 (via (at 91.5 92.5) (size 0.6) (drill 0.3) (layers "F.Cu" "B.Cu") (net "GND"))
 (via (at 96.75 81.75) (size 0.6) (drill 0.3) (layers "F.Cu" "B.Cu") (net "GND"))
 (via (at 90.25 94) (size 0.6) (drill 0.3) (layers "F.Cu" "B.Cu") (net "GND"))
 (via (at 82.25 85) (size 0.6) (drill 0.3) (layers "F.Cu" "B.Cu") (free yes) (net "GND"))
 (via (at 91.5 93.25) (size 0.6) (drill 0.3) (layers "F.Cu" "B.Cu") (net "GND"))
 (via (at 97.5 82.5) (size 0.6) (drill 0.3) (layers "F.Cu" "B.Cu") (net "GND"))
 (via (at 97.5 81.75) (size 0.6) (drill 0.3) (layers "F.Cu" "B.Cu") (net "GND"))
 (via (at 89 92.5) (size 0.6) (drill 0.3) (layers "F.Cu" "B.Cu") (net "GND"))
 (via (at 88.5 82.75) (size 0.6) (drill 0.3) (layers "F.Cu" "B.Cu") (free yes) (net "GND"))
 (via (at 89 94) (size 0.6) (drill 0.3) (layers "F.Cu" "B.Cu") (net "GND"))
 (via (at 87.5 83.5) (size 0.6) (drill 0.3) (layers "F.Cu" "B.Cu") (free yes) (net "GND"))
 (via (at 83.25 86) (size 0.6) (drill 0.3) (layers "F.Cu" "B.Cu") (free yes) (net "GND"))
 (via (at 96 82.5) (size 0.6) (drill 0.3) (layers "F.Cu" "B.Cu") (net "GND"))
 (via (at 96.75 82.5) (size 0.6) (drill 0.3) (layers "F.Cu" "B.Cu") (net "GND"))
 (via (at 91.5 94) (size 0.6) (drill 0.3) (layers "F.Cu" "B.Cu") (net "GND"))
 (segment (start 93.006823 81.506823) (end 94.522 83.022) (width 0.6) (layer "F.Cu") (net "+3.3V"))
 (segment (start 94.522 83.022) (end 94.522 86.698354) (width 0.6) (layer "F.Cu") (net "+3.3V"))
 (segment (start 88.1625 81.506823) (end 93.006823 81.506823) (width 0.6) (layer "F.Cu") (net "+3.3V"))
 (segment (start 86.195677 87.4125) (end 86.303177 87.305) (width 0.6) (layer "F.Cu") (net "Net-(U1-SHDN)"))
 (segment (start 84.496823 87.4125) (end 86.195677 87.4125) (width 0.6) (layer "F.Cu") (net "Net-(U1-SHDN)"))
 (segment (start 85.493177 81.506823) (end 86.3375 81.506823) (width 0.6) (layer "F.Cu") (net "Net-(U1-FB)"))
 (segment (start 86.3375 81.506823) (end 86.3375 84.960677) (width 0.6) (layer "F.Cu") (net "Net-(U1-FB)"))
 (segment (start 84.575 83.570677) (end 84.575 82.425) (width 0.6) (layer "F.Cu") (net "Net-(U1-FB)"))
 (segment (start 84.575 82.425) (end 85.493177 81.506823) (width 0.6) (layer "F.Cu") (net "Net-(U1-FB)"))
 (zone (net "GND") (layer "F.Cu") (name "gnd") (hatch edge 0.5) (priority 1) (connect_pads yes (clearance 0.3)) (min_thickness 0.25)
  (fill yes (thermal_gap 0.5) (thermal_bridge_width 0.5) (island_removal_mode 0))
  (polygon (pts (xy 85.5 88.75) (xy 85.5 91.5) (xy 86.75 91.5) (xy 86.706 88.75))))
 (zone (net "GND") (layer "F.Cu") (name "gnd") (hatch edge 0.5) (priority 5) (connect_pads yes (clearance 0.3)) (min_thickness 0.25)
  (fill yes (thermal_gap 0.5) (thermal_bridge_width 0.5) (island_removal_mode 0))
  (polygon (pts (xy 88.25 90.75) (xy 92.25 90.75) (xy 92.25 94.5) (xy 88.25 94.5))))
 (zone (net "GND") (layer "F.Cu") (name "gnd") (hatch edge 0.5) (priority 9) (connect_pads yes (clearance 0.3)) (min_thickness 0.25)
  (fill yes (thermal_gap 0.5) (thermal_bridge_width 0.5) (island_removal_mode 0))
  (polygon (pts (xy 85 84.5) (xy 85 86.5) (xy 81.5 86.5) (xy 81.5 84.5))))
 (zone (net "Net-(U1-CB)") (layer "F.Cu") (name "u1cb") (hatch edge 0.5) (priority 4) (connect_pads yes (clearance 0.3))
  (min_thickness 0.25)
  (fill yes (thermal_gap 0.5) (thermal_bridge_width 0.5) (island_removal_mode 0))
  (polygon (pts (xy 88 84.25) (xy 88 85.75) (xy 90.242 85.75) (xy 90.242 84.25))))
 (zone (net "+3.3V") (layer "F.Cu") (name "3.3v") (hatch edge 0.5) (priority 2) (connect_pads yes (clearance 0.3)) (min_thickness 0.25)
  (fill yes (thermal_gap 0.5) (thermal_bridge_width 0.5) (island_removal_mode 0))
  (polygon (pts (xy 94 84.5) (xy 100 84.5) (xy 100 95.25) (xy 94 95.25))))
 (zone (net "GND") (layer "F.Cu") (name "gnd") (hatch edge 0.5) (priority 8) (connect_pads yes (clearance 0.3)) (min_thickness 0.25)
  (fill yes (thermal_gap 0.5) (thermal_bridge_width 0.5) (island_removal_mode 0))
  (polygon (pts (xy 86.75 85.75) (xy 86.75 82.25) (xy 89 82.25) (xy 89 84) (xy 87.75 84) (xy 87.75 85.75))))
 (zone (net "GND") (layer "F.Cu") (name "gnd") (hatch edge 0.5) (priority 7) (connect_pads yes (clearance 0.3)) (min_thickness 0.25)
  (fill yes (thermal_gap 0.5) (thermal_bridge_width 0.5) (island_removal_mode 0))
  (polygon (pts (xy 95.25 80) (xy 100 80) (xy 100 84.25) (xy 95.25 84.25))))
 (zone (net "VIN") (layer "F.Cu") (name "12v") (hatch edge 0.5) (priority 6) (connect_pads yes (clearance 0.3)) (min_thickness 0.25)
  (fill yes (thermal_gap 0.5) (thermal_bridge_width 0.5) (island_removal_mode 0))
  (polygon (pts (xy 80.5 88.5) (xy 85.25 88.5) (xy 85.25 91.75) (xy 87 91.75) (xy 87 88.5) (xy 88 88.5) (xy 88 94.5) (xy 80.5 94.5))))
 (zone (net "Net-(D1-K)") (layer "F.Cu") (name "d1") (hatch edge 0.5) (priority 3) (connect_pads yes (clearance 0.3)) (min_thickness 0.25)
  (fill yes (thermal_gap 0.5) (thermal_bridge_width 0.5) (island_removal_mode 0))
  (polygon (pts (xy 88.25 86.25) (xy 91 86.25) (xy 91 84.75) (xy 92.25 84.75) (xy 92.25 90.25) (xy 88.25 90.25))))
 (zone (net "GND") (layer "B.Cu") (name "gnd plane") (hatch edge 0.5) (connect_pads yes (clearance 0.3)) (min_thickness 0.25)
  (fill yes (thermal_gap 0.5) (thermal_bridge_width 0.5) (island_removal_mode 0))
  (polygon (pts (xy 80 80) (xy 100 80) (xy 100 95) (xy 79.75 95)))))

